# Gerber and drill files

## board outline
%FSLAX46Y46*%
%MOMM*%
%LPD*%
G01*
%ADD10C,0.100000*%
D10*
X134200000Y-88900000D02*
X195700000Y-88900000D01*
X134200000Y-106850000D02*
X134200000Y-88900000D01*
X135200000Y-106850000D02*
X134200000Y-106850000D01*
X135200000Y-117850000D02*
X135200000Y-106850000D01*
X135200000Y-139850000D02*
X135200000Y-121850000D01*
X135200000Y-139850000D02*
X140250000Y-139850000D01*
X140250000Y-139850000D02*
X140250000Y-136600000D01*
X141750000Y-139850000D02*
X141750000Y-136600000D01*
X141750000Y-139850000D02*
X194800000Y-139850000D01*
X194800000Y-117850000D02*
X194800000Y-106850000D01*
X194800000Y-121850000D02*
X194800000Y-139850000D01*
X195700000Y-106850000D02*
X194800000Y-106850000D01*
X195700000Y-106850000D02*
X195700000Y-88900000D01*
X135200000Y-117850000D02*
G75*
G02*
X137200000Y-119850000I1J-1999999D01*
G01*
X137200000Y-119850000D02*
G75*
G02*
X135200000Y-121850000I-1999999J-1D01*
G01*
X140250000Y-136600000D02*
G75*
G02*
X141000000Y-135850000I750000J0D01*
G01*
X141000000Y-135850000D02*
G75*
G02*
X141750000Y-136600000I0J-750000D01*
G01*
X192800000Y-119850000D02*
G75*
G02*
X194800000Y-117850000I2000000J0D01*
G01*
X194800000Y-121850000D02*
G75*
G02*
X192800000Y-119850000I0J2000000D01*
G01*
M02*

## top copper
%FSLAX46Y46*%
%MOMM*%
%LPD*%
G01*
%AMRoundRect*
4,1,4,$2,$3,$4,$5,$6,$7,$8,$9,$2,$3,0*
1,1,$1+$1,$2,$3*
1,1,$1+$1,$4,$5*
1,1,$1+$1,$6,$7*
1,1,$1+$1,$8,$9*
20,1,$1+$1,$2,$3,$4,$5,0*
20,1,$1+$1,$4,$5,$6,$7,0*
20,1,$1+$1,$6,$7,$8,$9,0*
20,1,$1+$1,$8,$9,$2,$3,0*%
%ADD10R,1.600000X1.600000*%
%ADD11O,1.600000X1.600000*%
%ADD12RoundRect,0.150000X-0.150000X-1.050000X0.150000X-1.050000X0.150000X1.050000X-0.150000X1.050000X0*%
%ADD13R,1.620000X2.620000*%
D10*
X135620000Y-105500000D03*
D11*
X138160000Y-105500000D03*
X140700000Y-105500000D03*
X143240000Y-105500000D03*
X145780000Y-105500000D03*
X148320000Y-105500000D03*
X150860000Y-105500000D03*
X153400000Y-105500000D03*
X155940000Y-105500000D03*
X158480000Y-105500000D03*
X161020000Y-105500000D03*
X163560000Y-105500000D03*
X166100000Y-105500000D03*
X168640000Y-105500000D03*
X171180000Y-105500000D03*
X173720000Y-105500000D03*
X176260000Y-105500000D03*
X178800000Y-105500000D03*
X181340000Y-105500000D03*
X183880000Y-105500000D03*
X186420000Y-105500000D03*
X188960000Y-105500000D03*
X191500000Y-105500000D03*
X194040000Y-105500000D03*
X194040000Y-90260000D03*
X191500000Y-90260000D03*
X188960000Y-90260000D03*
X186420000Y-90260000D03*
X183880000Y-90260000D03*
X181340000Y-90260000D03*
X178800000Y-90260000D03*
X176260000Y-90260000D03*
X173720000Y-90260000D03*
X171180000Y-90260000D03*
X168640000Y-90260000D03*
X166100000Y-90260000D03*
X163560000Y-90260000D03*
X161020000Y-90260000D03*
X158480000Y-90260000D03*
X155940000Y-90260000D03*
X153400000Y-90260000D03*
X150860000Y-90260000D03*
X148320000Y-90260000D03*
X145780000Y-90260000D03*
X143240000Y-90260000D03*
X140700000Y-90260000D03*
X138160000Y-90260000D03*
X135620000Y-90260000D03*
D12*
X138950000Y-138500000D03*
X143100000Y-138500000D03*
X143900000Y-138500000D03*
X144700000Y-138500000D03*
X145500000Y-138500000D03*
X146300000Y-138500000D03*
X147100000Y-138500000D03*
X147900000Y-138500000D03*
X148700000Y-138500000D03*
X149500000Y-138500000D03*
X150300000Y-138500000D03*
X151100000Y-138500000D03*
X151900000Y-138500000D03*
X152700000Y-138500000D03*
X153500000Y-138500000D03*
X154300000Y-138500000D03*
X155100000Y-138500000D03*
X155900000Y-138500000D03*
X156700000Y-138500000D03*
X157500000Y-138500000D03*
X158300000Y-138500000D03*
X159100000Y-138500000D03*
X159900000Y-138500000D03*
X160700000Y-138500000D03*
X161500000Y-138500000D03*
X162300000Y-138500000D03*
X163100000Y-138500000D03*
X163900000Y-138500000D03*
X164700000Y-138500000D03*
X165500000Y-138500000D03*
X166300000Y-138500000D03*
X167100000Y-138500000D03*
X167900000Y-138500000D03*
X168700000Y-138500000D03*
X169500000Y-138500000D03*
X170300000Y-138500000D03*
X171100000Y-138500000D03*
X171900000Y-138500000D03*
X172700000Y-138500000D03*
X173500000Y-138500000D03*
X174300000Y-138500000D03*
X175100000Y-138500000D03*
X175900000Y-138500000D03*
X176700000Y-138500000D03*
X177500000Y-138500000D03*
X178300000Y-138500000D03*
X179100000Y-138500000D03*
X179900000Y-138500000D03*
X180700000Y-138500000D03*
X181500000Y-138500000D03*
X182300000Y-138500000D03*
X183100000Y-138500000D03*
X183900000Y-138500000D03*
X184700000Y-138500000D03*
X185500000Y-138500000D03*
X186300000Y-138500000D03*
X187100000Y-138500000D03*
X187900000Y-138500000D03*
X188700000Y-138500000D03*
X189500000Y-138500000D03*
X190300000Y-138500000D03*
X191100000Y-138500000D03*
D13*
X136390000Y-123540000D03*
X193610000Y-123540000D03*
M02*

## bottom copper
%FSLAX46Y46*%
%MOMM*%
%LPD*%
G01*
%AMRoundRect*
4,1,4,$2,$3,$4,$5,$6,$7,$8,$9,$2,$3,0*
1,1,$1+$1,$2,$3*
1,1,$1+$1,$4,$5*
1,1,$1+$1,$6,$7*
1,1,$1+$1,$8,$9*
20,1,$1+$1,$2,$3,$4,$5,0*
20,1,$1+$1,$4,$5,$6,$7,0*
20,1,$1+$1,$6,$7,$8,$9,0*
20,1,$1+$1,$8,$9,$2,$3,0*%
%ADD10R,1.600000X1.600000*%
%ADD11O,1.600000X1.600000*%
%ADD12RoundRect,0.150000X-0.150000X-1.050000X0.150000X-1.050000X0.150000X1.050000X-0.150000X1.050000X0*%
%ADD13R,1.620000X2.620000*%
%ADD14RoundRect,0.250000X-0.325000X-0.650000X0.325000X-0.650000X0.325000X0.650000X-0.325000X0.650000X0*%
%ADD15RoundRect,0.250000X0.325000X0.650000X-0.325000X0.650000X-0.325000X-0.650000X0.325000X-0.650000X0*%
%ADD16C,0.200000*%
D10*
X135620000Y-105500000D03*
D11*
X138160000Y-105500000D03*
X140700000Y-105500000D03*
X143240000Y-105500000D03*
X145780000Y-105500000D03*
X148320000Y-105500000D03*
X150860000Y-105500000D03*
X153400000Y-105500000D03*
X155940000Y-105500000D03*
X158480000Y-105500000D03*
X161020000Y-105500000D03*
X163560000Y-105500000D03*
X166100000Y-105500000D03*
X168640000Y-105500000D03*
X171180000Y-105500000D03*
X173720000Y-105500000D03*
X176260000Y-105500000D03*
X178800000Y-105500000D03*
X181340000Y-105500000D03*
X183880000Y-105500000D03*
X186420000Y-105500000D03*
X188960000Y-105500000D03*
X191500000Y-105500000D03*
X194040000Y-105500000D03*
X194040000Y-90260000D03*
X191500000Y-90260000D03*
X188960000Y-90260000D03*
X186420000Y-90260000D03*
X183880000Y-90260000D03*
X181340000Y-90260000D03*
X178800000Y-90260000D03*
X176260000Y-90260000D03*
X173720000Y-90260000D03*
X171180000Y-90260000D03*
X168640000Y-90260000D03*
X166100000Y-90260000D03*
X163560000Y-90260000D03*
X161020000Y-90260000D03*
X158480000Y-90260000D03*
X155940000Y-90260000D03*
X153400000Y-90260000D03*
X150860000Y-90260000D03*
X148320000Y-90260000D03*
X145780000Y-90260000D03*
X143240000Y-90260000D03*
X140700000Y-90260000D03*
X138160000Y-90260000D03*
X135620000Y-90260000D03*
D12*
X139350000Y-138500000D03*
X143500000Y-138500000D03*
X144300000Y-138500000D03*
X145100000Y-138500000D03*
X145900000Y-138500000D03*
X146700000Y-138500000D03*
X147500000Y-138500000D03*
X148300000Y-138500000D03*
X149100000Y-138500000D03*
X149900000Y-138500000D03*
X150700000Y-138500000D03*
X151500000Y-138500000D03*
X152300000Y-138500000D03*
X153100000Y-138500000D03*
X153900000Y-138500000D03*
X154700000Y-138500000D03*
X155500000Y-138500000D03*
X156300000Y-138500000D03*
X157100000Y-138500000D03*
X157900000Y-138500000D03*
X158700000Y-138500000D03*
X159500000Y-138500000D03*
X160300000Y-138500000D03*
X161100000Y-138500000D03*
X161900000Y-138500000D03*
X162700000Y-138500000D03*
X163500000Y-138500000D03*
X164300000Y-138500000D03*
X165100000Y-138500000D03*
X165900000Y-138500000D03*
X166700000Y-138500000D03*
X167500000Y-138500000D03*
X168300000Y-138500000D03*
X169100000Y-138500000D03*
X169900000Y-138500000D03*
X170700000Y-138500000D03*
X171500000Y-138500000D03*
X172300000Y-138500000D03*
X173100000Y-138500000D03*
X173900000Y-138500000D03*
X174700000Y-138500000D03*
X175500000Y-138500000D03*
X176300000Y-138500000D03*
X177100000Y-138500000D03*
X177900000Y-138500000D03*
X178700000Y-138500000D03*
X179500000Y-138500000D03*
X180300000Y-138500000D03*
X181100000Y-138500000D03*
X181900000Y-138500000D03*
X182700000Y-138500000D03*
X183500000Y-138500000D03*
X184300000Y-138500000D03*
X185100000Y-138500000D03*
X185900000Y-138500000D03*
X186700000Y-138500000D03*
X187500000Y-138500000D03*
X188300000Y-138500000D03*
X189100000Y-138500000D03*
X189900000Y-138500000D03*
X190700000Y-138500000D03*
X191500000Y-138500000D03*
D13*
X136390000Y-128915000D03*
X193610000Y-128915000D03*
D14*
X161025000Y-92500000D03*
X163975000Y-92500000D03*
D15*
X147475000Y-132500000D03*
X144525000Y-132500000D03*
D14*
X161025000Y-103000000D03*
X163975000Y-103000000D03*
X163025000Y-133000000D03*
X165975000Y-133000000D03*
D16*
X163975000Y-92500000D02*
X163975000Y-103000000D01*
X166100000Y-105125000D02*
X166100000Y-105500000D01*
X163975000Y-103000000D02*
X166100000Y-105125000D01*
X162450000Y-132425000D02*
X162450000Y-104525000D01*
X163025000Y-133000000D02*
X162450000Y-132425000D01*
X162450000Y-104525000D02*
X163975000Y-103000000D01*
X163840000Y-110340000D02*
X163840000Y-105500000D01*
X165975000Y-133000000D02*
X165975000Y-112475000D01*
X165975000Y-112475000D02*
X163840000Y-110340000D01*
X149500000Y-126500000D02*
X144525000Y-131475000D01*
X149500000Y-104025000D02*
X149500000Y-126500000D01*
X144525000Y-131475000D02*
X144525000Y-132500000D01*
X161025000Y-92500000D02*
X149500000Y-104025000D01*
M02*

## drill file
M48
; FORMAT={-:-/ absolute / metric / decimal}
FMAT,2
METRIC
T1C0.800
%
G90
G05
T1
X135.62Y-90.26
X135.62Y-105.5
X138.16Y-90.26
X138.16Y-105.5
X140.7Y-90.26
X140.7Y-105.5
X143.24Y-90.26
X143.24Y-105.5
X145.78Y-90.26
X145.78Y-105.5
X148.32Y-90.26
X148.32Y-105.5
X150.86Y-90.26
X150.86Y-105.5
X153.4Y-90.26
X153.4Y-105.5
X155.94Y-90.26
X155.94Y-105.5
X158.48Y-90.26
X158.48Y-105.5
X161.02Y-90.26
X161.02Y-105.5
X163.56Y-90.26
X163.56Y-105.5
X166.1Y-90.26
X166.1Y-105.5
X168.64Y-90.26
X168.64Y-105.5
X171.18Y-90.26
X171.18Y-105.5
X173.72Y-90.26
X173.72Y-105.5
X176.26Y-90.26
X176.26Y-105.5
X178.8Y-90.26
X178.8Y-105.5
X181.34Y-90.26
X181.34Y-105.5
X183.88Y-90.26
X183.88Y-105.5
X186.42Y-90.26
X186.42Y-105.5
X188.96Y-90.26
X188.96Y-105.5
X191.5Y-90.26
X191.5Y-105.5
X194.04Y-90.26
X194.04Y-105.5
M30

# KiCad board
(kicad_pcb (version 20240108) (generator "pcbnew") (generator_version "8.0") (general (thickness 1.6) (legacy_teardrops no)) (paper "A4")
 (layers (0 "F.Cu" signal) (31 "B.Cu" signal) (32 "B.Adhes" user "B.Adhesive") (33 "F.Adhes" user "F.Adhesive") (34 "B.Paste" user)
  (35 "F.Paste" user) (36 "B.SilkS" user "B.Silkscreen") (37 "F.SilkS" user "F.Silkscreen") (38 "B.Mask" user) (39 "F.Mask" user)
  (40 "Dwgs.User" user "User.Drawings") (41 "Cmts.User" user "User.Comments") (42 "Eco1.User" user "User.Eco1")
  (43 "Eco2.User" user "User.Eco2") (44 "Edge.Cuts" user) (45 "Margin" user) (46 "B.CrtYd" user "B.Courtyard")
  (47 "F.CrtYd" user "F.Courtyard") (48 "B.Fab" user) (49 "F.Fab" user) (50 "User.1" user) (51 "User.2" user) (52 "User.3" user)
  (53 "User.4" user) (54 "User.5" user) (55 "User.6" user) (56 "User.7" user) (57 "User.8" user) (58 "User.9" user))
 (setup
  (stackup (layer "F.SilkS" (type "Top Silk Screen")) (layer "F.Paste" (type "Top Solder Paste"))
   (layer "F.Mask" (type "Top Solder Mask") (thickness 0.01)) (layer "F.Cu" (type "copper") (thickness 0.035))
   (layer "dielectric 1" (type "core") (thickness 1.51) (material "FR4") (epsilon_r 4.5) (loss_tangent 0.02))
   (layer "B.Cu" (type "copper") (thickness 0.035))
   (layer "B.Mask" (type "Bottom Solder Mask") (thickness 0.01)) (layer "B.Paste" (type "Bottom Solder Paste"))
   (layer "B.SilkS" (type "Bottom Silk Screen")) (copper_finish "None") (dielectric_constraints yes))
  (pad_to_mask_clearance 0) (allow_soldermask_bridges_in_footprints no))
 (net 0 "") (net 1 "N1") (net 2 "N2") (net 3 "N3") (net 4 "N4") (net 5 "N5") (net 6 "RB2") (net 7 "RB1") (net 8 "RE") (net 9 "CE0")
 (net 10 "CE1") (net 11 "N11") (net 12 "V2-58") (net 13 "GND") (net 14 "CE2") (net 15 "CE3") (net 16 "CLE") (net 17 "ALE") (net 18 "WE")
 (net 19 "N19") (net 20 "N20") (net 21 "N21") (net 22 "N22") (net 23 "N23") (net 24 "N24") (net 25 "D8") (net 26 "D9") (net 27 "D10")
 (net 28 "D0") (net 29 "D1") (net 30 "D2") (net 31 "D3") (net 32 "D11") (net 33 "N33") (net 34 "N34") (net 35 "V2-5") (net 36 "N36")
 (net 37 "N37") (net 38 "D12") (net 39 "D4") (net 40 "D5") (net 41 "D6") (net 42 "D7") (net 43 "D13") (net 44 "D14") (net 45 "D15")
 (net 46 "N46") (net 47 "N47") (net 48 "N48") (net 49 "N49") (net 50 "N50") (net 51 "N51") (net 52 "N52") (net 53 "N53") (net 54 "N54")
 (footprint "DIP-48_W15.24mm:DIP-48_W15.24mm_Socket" (layer "F.Cu") (at 135.62 105.5 90)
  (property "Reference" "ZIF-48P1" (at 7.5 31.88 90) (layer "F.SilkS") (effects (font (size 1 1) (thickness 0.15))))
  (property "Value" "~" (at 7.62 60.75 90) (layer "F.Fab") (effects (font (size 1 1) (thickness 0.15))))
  (pad "1" thru_hole rect (at 0 0 90) (size 1.6 1.6) (drill 0.8) (layers "*.Cu" "*.Mask") (remove_unused_layers no) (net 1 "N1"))
  (pad "2" thru_hole oval (at 0 2.54 90) (size 1.6 1.6) (drill 0.8) (layers "*.Cu" "*.Mask") (remove_unused_layers no) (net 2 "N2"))
  (pad "3" thru_hole oval (at 0 5.08 90) (size 1.6 1.6) (drill 0.8) (layers "*.Cu" "*.Mask") (remove_unused_layers no) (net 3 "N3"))
  (pad "4" thru_hole oval (at 0 7.62 90) (size 1.6 1.6) (drill 0.8) (layers "*.Cu" "*.Mask") (remove_unused_layers no) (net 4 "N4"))
  (pad "5" thru_hole oval (at 0 10.16 90) (size 1.6 1.6) (drill 0.8) (layers "*.Cu" "*.Mask") (remove_unused_layers no) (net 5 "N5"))
  (pad "6" thru_hole oval (at 0 12.7 90) (size 1.6 1.6) (drill 0.8) (layers "*.Cu" "*.Mask") (remove_unused_layers no) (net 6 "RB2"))
  (pad "7" thru_hole oval (at 0 15.24 90) (size 1.6 1.6) (drill 0.8) (layers "*.Cu" "*.Mask") (remove_unused_layers no) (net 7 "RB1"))
  (pad "8" thru_hole oval (at 0 17.78 90) (size 1.6 1.6) (drill 0.8) (layers "*.Cu" "*.Mask") (remove_unused_layers no) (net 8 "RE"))
  (pad "9" thru_hole oval (at 0 20.32 90) (size 1.6 1.6) (drill 0.8) (layers "*.Cu" "*.Mask") (remove_unused_layers no) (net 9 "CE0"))
  (pad "10" thru_hole oval (at 0 22.86 90) (size 1.6 1.6) (drill 0.8) (layers "*.Cu" "*.Mask") (remove_unused_layers no) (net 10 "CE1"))
  (pad "11" thru_hole oval (at 0 25.4 90) (size 1.6 1.6) (drill 0.8) (layers "*.Cu" "*.Mask") (remove_unused_layers no) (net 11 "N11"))
  (pad "12" thru_hole oval (at 0 27.94 90) (size 1.6 1.6) (drill 0.8) (layers "*.Cu" "*.Mask") (remove_unused_layers no) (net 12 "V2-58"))
  (pad "13" thru_hole oval (at 0 30.48 90) (size 1.6 1.6) (drill 0.8) (layers "*.Cu" "*.Mask") (remove_unused_layers no) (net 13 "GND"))
  (pad "14" thru_hole oval (at 0 33.02 90) (size 1.6 1.6) (drill 0.8) (layers "*.Cu" "*.Mask") (remove_unused_layers no) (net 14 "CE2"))
  (pad "15" thru_hole oval (at 0 35.56 90) (size 1.6 1.6) (drill 0.8) (layers "*.Cu" "*.Mask") (remove_unused_layers no) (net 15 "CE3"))
  (pad "16" thru_hole oval (at 0 38.1 90) (size 1.6 1.6) (drill 0.8) (layers "*.Cu" "*.Mask") (remove_unused_layers no) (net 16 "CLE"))
  (pad "17" thru_hole oval (at 0 40.64 90) (size 1.6 1.6) (drill 0.8) (layers "*.Cu" "*.Mask") (remove_unused_layers no) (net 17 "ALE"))
  (pad "18" thru_hole oval (at 0 43.18 90) (size 1.6 1.6) (drill 0.8) (layers "*.Cu" "*.Mask") (remove_unused_layers no) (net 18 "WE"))
  (pad "19" thru_hole oval (at 0 45.72 90) (size 1.6 1.6) (drill 0.8) (layers "*.Cu" "*.Mask") (remove_unused_layers no) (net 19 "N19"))
  (pad "20" thru_hole oval (at 0 48.26 90) (size 1.6 1.6) (drill 0.8) (layers "*.Cu" "*.Mask") (remove_unused_layers no) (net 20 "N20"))
  (pad "21" thru_hole oval (at 0 50.8 90) (size 1.6 1.6) (drill 0.8) (layers "*.Cu" "*.Mask") (remove_unused_layers no) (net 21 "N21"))
  (pad "22" thru_hole oval (at 0 53.34 90) (size 1.6 1.6) (drill 0.8) (layers "*.Cu" "*.Mask") (remove_unused_layers no) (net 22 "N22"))
  (pad "23" thru_hole oval (at 0 55.88 90) (size 1.6 1.6) (drill 0.8) (layers "*.Cu" "*.Mask") (remove_unused_layers no) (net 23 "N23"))
  (pad "24" thru_hole oval (at 0 58.42 90) (size 1.6 1.6) (drill 0.8) (layers "*.Cu" "*.Mask") (remove_unused_layers no) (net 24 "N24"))
  (pad "25" thru_hole oval (at 15.24 58.42 90) (size 1.6 1.6) (drill 0.8) (layers "*.Cu" "*.Mask") (remove_unused_layers no) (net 13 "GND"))
  (pad "26" thru_hole oval (at 15.24 55.88 90) (size 1.6 1.6) (drill 0.8) (layers "*.Cu" "*.Mask") (remove_unused_layers no) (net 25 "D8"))
  (pad "27" thru_hole oval (at 15.24 53.34 90) (size 1.6 1.6) (drill 0.8) (layers "*.Cu" "*.Mask") (remove_unused_layers no) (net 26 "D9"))
  (pad "28" thru_hole oval (at 15.24 50.8 90) (size 1.6 1.6) (drill 0.8) (layers "*.Cu" "*.Mask") (remove_unused_layers no) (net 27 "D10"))
  (pad "29" thru_hole oval (at 15.24 48.26 90) (size 1.6 1.6) (drill 0.8) (layers "*.Cu" "*.Mask") (remove_unused_layers no) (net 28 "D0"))
  (pad "30" thru_hole oval (at 15.24 45.72 90) (size 1.6 1.6) (drill 0.8) (layers "*.Cu" "*.Mask") (remove_unused_layers no) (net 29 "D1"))
  (pad "31" thru_hole oval (at 15.24 43.18 90) (size 1.6 1.6) (drill 0.8) (layers "*.Cu" "*.Mask") (remove_unused_layers no) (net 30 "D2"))
  (pad "32" thru_hole oval (at 15.24 40.64 90) (size 1.6 1.6) (drill 0.8) (layers "*.Cu" "*.Mask") (remove_unused_layers no) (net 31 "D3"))
  (pad "33" thru_hole oval (at 15.24 38.1 90) (size 1.6 1.6) (drill 0.8) (layers "*.Cu" "*.Mask") (remove_unused_layers no) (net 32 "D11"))
  (pad "34" thru_hole oval (at 15.24 35.56 90) (size 1.6 1.6) (drill 0.8) (layers "*.Cu" "*.Mask") (remove_unused_layers no) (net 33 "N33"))
  (pad "35" thru_hole oval (at 15.24 33.02 90) (size 1.6 1.6) (drill 0.8) (layers "*.Cu" "*.Mask") (remove_unused_layers no) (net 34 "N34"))
  (pad "36" thru_hole oval (at 15.24 30.48 90) (size 1.6 1.6) (drill 0.8) (layers "*.Cu" "*.Mask") (remove_unused_layers no) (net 13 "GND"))
  (pad "37" thru_hole oval (at 15.24 27.94 90) (size 1.6 1.6) (drill 0.8) (layers "*.Cu" "*.Mask") (remove_unused_layers no) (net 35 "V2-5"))
  (pad "38" thru_hole oval (at 15.24 25.4 90) (size 1.6 1.6) (drill 0.8) (layers "*.Cu" "*.Mask") (remove_unused_layers no) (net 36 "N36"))
  (pad "39" thru_hole oval (at 15.24 22.86 90) (size 1.6 1.6) (drill 0.8) (layers "*.Cu" "*.Mask") (remove_unused_layers no) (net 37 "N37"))
  (pad "40" thru_hole oval (at 15.24 20.32 90) (size 1.6 1.6) (drill 0.8) (layers "*.Cu" "*.Mask") (remove_unused_layers no) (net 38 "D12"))
  (pad "41" thru_hole oval (at 15.24 17.78 90) (size 1.6 1.6) (drill 0.8) (layers "*.Cu" "*.Mask") (remove_unused_layers no) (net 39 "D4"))
  (pad "42" thru_hole oval (at 15.24 15.24 90) (size 1.6 1.6) (drill 0.8) (layers "*.Cu" "*.Mask") (remove_unused_layers no) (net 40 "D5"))
  (pad "43" thru_hole oval (at 15.24 12.7 90) (size 1.6 1.6) (drill 0.8) (layers "*.Cu" "*.Mask") (remove_unused_layers no) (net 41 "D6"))
  (pad "44" thru_hole oval (at 15.24 10.16 90) (size 1.6 1.6) (drill 0.8) (layers "*.Cu" "*.Mask") (remove_unused_layers no) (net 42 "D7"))
  (pad "45" thru_hole oval (at 15.24 7.62 90) (size 1.6 1.6) (drill 0.8) (layers "*.Cu" "*.Mask") (remove_unused_layers no) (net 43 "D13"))
  (pad "46" thru_hole oval (at 15.24 5.08 90) (size 1.6 1.6) (drill 0.8) (layers "*.Cu" "*.Mask") (remove_unused_layers no) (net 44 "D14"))
  (pad "47" thru_hole oval (at 15.24 2.54 90) (size 1.6 1.6) (drill 0.8) (layers "*.Cu" "*.Mask") (remove_unused_layers no) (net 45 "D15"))
  (pad "48" thru_hole oval (at 15.24 0 90) (size 1.6 1.6) (drill 0.8) (layers "*.Cu" "*.Mask") (remove_unused_layers no) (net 13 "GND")))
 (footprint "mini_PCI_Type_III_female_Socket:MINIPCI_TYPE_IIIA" (layer "F.Cu") (at 135.2 139.85)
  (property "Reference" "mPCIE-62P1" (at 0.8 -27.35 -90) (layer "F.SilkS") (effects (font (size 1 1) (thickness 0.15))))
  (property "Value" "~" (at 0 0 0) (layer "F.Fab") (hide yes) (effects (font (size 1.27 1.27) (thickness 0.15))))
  (fp_line (start -1 -50.95) (end 60.5 -50.95) (stroke (width 0.1) (type solid)) (layer "Edge.Cuts"))
  (fp_line (start -1 -33) (end -1 -50.95) (stroke (width 0.1) (type solid)) (layer "Edge.Cuts"))
  (fp_line (start 0 -33) (end -1 -33) (stroke (width 0.1) (type solid)) (layer "Edge.Cuts"))
  (fp_line (start 0 -22) (end 0 -33) (stroke (width 0.1) (type solid)) (layer "Edge.Cuts"))
  (fp_line (start 0 0) (end 0 -18) (stroke (width 0.1) (type solid)) (layer "Edge.Cuts"))
  (fp_line (start 0 0) (end 5.05 0) (stroke (width 0.1) (type solid)) (layer "Edge.Cuts"))
  (fp_line (start 5.05 0) (end 5.05 -3.25) (stroke (width 0.1) (type solid)) (layer "Edge.Cuts"))
  (fp_line (start 6.55 0) (end 6.55 -3.25) (stroke (width 0.1) (type solid)) (layer "Edge.Cuts"))
  (fp_line (start 6.55 0) (end 59.6 0) (stroke (width 0.1) (type solid)) (layer "Edge.Cuts"))
  (fp_line (start 59.6 -22) (end 59.6 -33) (stroke (width 0.1) (type solid)) (layer "Edge.Cuts"))
  (fp_line (start 59.6 -18) (end 59.6 0) (stroke (width 0.1) (type solid)) (layer "Edge.Cuts"))
  (fp_line (start 60.5 -33) (end 59.6 -33) (stroke (width 0.1) (type solid)) (layer "Edge.Cuts"))
  (fp_line (start 60.5 -33) (end 60.5 -50.95) (stroke (width 0.1) (type solid)) (layer "Edge.Cuts"))
  (fp_arc (start 0 -22) (mid 1.414214 -21.414214) (end 2 -20) (stroke (width 0.1) (type solid)) (layer "Edge.Cuts"))
  (fp_arc (start 2 -20) (mid 1.414214 -18.585786) (end 0 -18) (stroke (width 0.1) (type solid)) (layer "Edge.Cuts"))
  (fp_arc (start 5.05 -3.25) (mid 5.26967 -3.78033) (end 5.8 -4) (stroke (width 0.1) (type solid)) (layer "Edge.Cuts"))
  (fp_arc (start 5.8 -4) (mid 6.33033 -3.78033) (end 6.55 -3.25) (stroke (width 0.1) (type solid)) (layer "Edge.Cuts"))
  (fp_arc (start 57.6 -20) (mid 58.185786 -21.414214) (end 59.6 -22) (stroke (width 0.1) (type solid)) (layer "Edge.Cuts"))
  (fp_arc (start 59.6 -18) (mid 58.185786 -18.585786) (end 57.6 -20) (stroke (width 0.1) (type solid)) (layer "Edge.Cuts"))
  (pad "1" smd roundrect (at 3.75 -1.35) (size 0.6 2.4) (layers "F.Cu") (roundrect_rratio 0.25) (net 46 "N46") (solder_mask_margin 0.1016)
   (thermal_bridge_angle 0))
  (pad "1" smd roundrect (at 4.15 -1.35) (size 0.6 2.4) (layers "B.Cu") (roundrect_rratio 0.25) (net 46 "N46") (solder_mask_margin 0.1016)
   (thermal_bridge_angle 0))
  (pad "2" smd roundrect (at 7.9 -1.35) (size 0.6 2.4) (layers "F.Cu") (roundrect_rratio 0.25) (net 2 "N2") (solder_mask_margin 0.1016)
   (thermal_bridge_angle 0))
  (pad "2" smd roundrect (at 8.3 -1.35) (size 0.6 2.4) (layers "B.Cu") (roundrect_rratio 0.25) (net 2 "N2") (solder_mask_margin 0.1016)
   (thermal_bridge_angle 0))
  (pad "3" smd roundrect (at 8.7 -1.35) (size 0.6 2.4) (layers "F.Cu") (roundrect_rratio 0.25) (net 3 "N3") (solder_mask_margin 0.1016)
   (thermal_bridge_angle 0))
  (pad "3" smd roundrect (at 9.1 -1.35) (size 0.6 2.4) (layers "B.Cu") (roundrect_rratio 0.25) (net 3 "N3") (solder_mask_margin 0.1016)
   (thermal_bridge_angle 0))
  (pad "4" smd roundrect (at 9.5 -1.35) (size 0.6 2.4) (layers "F.Cu") (roundrect_rratio 0.25) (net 4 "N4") (solder_mask_margin 0.1016)
   (thermal_bridge_angle 0))
  (pad "4" smd roundrect (at 9.9 -1.35) (size 0.6 2.4) (layers "B.Cu") (roundrect_rratio 0.25) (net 4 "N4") (solder_mask_margin 0.1016)
   (thermal_bridge_angle 0))
  (pad "5" smd roundrect (at 10.3 -1.35) (size 0.6 2.4) (layers "F.Cu") (roundrect_rratio 0.25) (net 35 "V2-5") (solder_mask_margin 0.1016)
   (thermal_bridge_angle 0))
  (pad "5" smd roundrect (at 10.7 -1.35) (size 0.6 2.4) (layers "B.Cu") (roundrect_rratio 0.25) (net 35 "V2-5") (solder_mask_margin 0.1016)
   (thermal_bridge_angle 0))
  (pad "6" smd roundrect (at 11.1 -1.35) (size 0.6 2.4) (layers "F.Cu") (roundrect_rratio 0.25) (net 13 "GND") (solder_mask_margin 0.1016)
   (thermal_bridge_angle 0))
  (pad "6" smd roundrect (at 11.5 -1.35) (size 0.6 2.4) (layers "B.Cu") (roundrect_rratio 0.25) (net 13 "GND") (solder_mask_margin 0.1016)
   (thermal_bridge_angle 0))
  (pad "7" smd roundrect (at 11.9 -1.35) (size 0.6 2.4) (layers "F.Cu") (roundrect_rratio 0.25) (solder_mask_margin 0.1016)
   (thermal_bridge_angle 0))
  (pad "7" smd roundrect (at 12.3 -1.35) (size 0.6 2.4) (layers "B.Cu") (roundrect_rratio 0.25) (solder_mask_margin 0.1016)
   (thermal_bridge_angle 0))
  (pad "8" smd roundrect (at 12.7 -1.35) (size 0.6 2.4) (layers "F.Cu") (roundrect_rratio 0.25) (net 13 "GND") (solder_mask_margin 0.1016)
   (thermal_bridge_angle 0))
  (pad "8" smd roundrect (at 13.1 -1.35) (size 0.6 2.4) (layers "B.Cu") (roundrect_rratio 0.25) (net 13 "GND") (solder_mask_margin 0.1016)
   (thermal_bridge_angle 0))
  (pad "9" smd roundrect (at 13.5 -1.35) (size 0.6 2.4) (layers "F.Cu") (roundrect_rratio 0.25) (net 13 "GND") (solder_mask_margin 0.1016)
   (thermal_bridge_angle 0))
  (pad "9" smd roundrect (at 13.9 -1.35) (size 0.6 2.4) (layers "B.Cu") (roundrect_rratio 0.25) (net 13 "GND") (solder_mask_margin 0.1016)
   (thermal_bridge_angle 0))
  (pad "10" smd roundrect (at 14.3 -1.35) (size 0.6 2.4) (layers "F.Cu") (roundrect_rratio 0.25) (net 13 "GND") (solder_mask_margin 0.1016)
   (thermal_bridge_angle 0))
  (pad "10" smd roundrect (at 14.7 -1.35) (size 0.6 2.4) (layers "B.Cu") (roundrect_rratio 0.25) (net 13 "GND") (solder_mask_margin 0.1016)
   (thermal_bridge_angle 0))
  (pad "11" smd roundrect (at 15.1 -1.35) (size 0.6 2.4) (layers "F.Cu") (roundrect_rratio 0.25) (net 11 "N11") (solder_mask_margin 0.1016)
   (thermal_bridge_angle 0))
  (pad "11" smd roundrect (at 15.5 -1.35) (size 0.6 2.4) (layers "B.Cu") (roundrect_rratio 0.25) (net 11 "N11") (solder_mask_margin 0.1016)
   (thermal_bridge_angle 0))
  (pad "12" smd roundrect (at 15.9 -1.35) (size 0.6 2.4) (layers "F.Cu") (roundrect_rratio 0.25) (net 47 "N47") (solder_mask_margin 0.1016)
   (thermal_bridge_angle 0))
  (pad "12" smd roundrect (at 16.3 -1.35) (size 0.6 2.4) (layers "B.Cu") (roundrect_rratio 0.25) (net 47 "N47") (solder_mask_margin 0.1016)
   (thermal_bridge_angle 0))
  (pad "13" smd roundrect (at 16.7 -1.35) (size 0.6 2.4) (layers "F.Cu") (roundrect_rratio 0.25) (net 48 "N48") (solder_mask_margin 0.1016)
   (thermal_bridge_angle 0))
  (pad "13" smd roundrect (at 17.1 -1.35) (size 0.6 2.4) (layers "B.Cu") (roundrect_rratio 0.25) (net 48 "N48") (solder_mask_margin 0.1016)
   (thermal_bridge_angle 0))
  (pad "14" smd roundrect (at 17.5 -1.35) (size 0.6 2.4) (layers "F.Cu") (roundrect_rratio 0.25) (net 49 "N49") (solder_mask_margin 0.1016)
   (thermal_bridge_angle 0))
  (pad "14" smd roundrect (at 17.9 -1.35) (size 0.6 2.4) (layers "B.Cu") (roundrect_rratio 0.25) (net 49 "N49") (solder_mask_margin 0.1016)
   (thermal_bridge_angle 0))
  (pad "15" smd roundrect (at 18.3 -1.35) (size 0.6 2.4) (layers "F.Cu") (roundrect_rratio 0.25) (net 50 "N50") (solder_mask_margin 0.1016)
   (thermal_bridge_angle 0))
  (pad "15" smd roundrect (at 18.7 -1.35) (size 0.6 2.4) (layers "B.Cu") (roundrect_rratio 0.25) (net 50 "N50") (solder_mask_margin 0.1016)
   (thermal_bridge_angle 0))
  (pad "16" smd roundrect (at 19.1 -1.35) (size 0.6 2.4) (layers "F.Cu") (roundrect_rratio 0.25) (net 13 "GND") (solder_mask_margin 0.1016)
   (thermal_bridge_angle 0))
  (pad "16" smd roundrect (at 19.5 -1.35) (size 0.6 2.4) (layers "B.Cu") (roundrect_rratio 0.25) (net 13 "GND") (solder_mask_margin 0.1016)
   (thermal_bridge_angle 0))
  (pad "17" smd roundrect (at 19.9 -1.35) (size 0.6 2.4) (layers "F.Cu") (roundrect_rratio 0.25) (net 27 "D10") (solder_mask_margin 0.1016)
   (thermal_bridge_angle 0))
  (pad "17" smd roundrect (at 20.3 -1.35) (size 0.6 2.4) (layers "B.Cu") (roundrect_rratio 0.25) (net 27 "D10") (solder_mask_margin 0.1016)
   (thermal_bridge_angle 0))
  (pad "18" smd roundrect (at 20.7 -1.35) (size 0.6 2.4) (layers "F.Cu") (roundrect_rratio 0.25) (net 30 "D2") (solder_mask_margin 0.1016)
   (thermal_bridge_angle 0))
  (pad "18" smd roundrect (at 21.1 -1.35) (size 0.6 2.4) (layers "B.Cu") (roundrect_rratio 0.25) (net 30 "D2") (solder_mask_margin 0.1016)
   (thermal_bridge_angle 0))
  (pad "19" smd roundrect (at 21.5 -1.35) (size 0.6 2.4) (layers "F.Cu") (roundrect_rratio 0.25) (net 13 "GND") (solder_mask_margin 0.1016)
   (thermal_bridge_angle 0))
  (pad "19" smd roundrect (at 21.9 -1.35) (size 0.6 2.4) (layers "B.Cu") (roundrect_rratio 0.25) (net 13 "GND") (solder_mask_margin 0.1016)
   (thermal_bridge_angle 0))
  (pad "20" smd roundrect (at 22.3 -1.35) (size 0.6 2.4) (layers "F.Cu") (roundrect_rratio 0.25) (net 32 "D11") (solder_mask_margin 0.1016)
   (thermal_bridge_angle 0))
  (pad "20" smd roundrect (at 22.7 -1.35) (size 0.6 2.4) (layers "B.Cu") (roundrect_rratio 0.25) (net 32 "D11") (solder_mask_margin 0.1016)
   (thermal_bridge_angle 0))
  (pad "21" smd roundrect (at 23.1 -1.35) (size 0.6 2.4) (layers "F.Cu") (roundrect_rratio 0.25) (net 29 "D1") (solder_mask_margin 0.1016)
   (thermal_bridge_angle 0))
  (pad "21" smd roundrect (at 23.5 -1.35) (size 0.6 2.4) (layers "B.Cu") (roundrect_rratio 0.25) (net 29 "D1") (solder_mask_margin 0.1016)
   (thermal_bridge_angle 0))
  (pad "22" smd roundrect (at 23.9 -1.35) (size 0.6 2.4) (layers "F.Cu") (roundrect_rratio 0.25) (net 13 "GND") (solder_mask_margin 0.1016)
   (thermal_bridge_angle 0))
  (pad "22" smd roundrect (at 24.3 -1.35) (size 0.6 2.4) (layers "B.Cu") (roundrect_rratio 0.25) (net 13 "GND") (solder_mask_margin 0.1016)
   (thermal_bridge_angle 0))
  (pad "23" smd roundrect (at 24.7 -1.35) (size 0.6 2.4) (layers "F.Cu") (roundrect_rratio 0.25) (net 25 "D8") (solder_mask_margin 0.1016)
   (thermal_bridge_angle 0))
  (pad "23" smd roundrect (at 25.1 -1.35) (size 0.6 2.4) (layers "B.Cu") (roundrect_rratio 0.25) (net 25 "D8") (solder_mask_margin 0.1016)
   (thermal_bridge_angle 0))
  (pad "24" smd roundrect (at 25.5 -1.35) (size 0.6 2.4) (layers "F.Cu") (roundrect_rratio 0.25) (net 26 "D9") (solder_mask_margin 0.1016)
   (thermal_bridge_angle 0))
  (pad "24" smd roundrect (at 25.9 -1.35) (size 0.6 2.4) (layers "B.Cu") (roundrect_rratio 0.25) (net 26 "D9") (solder_mask_margin 0.1016)
   (thermal_bridge_angle 0))
  (pad "25" smd roundrect (at 26.3 -1.35) (size 0.6 2.4) (layers "F.Cu") (roundrect_rratio 0.25) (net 13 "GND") (solder_mask_margin 0.1016)
   (thermal_bridge_angle 0))
  (pad "25" smd roundrect (at 26.7 -1.35) (size 0.6 2.4) (layers "B.Cu") (roundrect_rratio 0.25) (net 13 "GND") (solder_mask_margin 0.1016)
   (thermal_bridge_angle 0))
  (pad "26" smd roundrect (at 27.1 -1.35) (size 0.6 2.4) (layers "F.Cu") (roundrect_rratio 0.25) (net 31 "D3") (solder_mask_margin 0.1016)
   (thermal_bridge_angle 0))
  (pad "26" smd roundrect (at 27.5 -1.35) (size 0.6 2.4) (layers "B.Cu") (roundrect_rratio 0.25) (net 31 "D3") (solder_mask_margin 0.1016)
   (thermal_bridge_angle 0))
  (pad "27" smd roundrect (at 27.9 -1.35) (size 0.6 2.4) (layers "F.Cu") (roundrect_rratio 0.25) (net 28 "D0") (solder_mask_margin 0.1016)
   (thermal_bridge_angle 0))
  (pad "27" smd roundrect (at 28.3 -1.35) (size 0.6 2.4) (layers "B.Cu") (roundrect_rratio 0.25) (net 28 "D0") (solder_mask_margin 0.1016)
   (thermal_bridge_angle 0))
  (pad "28" smd roundrect (at 28.7 -1.35) (size 0.6 2.4) (layers "F.Cu") (roundrect_rratio 0.25) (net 13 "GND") (solder_mask_margin 0.1016)
   (thermal_bridge_angle 0))
  (pad "28" smd roundrect (at 29.1 -1.35) (size 0.6 2.4) (layers "B.Cu") (roundrect_rratio 0.25) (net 13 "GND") (solder_mask_margin 0.1016)
   (thermal_bridge_angle 0))
  (pad "29" smd roundrect (at 29.5 -1.35) (size 0.6 2.4) (layers "F.Cu") (roundrect_rratio 0.25) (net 18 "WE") (solder_mask_margin 0.1016)
   (thermal_bridge_angle 0))
  (pad "29" smd roundrect (at 29.9 -1.35) (size 0.6 2.4) (layers "B.Cu") (roundrect_rratio 0.25) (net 18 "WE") (solder_mask_margin 0.1016)
   (thermal_bridge_angle 0))
  (pad "30" smd roundrect (at 30.3 -1.35) (size 0.6 2.4) (layers "F.Cu") (roundrect_rratio 0.25) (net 13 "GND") (solder_mask_margin 0.1016)
   (thermal_bridge_angle 0))
  (pad "30" smd roundrect (at 30.7 -1.35) (size 0.6 2.4) (layers "B.Cu") (roundrect_rratio 0.25) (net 13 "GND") (solder_mask_margin 0.1016)
   (thermal_bridge_angle 0))
  (pad "31" smd roundrect (at 31.1 -1.35) (size 0.6 2.4) (layers "F.Cu") (roundrect_rratio 0.25) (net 16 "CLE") (solder_mask_margin 0.1016)
   (thermal_bridge_angle 0))
  (pad "31" smd roundrect (at 31.5 -1.35) (size 0.6 2.4) (layers "B.Cu") (roundrect_rratio 0.25) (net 16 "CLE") (solder_mask_margin 0.1016)
   (thermal_bridge_angle 0))
  (pad "32" smd roundrect (at 31.9 -1.35) (size 0.6 2.4) (layers "F.Cu") (roundrect_rratio 0.25) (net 13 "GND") (solder_mask_margin 0.1016)
   (thermal_bridge_angle 0))
  (pad "32" smd roundrect (at 32.3 -1.35) (size 0.6 2.4) (layers "B.Cu") (roundrect_rratio 0.25) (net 13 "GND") (solder_mask_margin 0.1016)
   (thermal_bridge_angle 0))
  (pad "33" smd roundrect (at 32.7 -1.35) (size 0.6 2.4) (layers "F.Cu") (roundrect_rratio 0.25) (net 17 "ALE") (solder_mask_margin 0.1016)
   (thermal_bridge_angle 0))
  (pad "33" smd roundrect (at 33.1 -1.35) (size 0.6 2.4) (layers "B.Cu") (roundrect_rratio 0.25) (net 17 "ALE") (solder_mask_margin 0.1016)
   (thermal_bridge_angle 0))
  (pad "34" smd roundrect (at 33.5 -1.35) (size 0.6 2.4) (layers "F.Cu") (roundrect_rratio 0.25) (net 13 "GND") (solder_mask_margin 0.1016)
   (thermal_bridge_angle 0))
  (pad "34" smd roundrect (at 33.9 -1.35) (size 0.6 2.4) (layers "B.Cu") (roundrect_rratio 0.25) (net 13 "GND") (solder_mask_margin 0.1016)
   (thermal_bridge_angle 0))
  (pad "35" smd roundrect (at 34.3 -1.35) (size 0.6 2.4) (layers "F.Cu") (roundrect_rratio 0.25) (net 9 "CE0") (solder_mask_margin 0.1016)
   (thermal_bridge_angle 0))
  (pad "35" smd roundrect (at 34.7 -1.35) (size 0.6 2.4) (layers "B.Cu") (roundrect_rratio 0.25) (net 9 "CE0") (solder_mask_margin 0.1016)
   (thermal_bridge_angle 0))
  (pad "36" smd roundrect (at 35.1 -1.35) (size 0.6 2.4) (layers "F.Cu") (roundrect_rratio 0.25) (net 14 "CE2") (solder_mask_margin 0.1016)
   (thermal_bridge_angle 0))
  (pad "36" smd roundrect (at 35.5 -1.35) (size 0.6 2.4) (layers "B.Cu") (roundrect_rratio 0.25) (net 14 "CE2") (solder_mask_margin 0.1016)
   (thermal_bridge_angle 0))
  (pad "37" smd roundrect (at 35.9 -1.35) (size 0.6 2.4) (layers "F.Cu") (roundrect_rratio 0.25) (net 10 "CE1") (solder_mask_margin 0.1016)
   (thermal_bridge_angle 0))
  (pad "37" smd roundrect (at 36.3 -1.35) (size 0.6 2.4) (layers "B.Cu") (roundrect_rratio 0.25) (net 10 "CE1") (solder_mask_margin 0.1016)
   (thermal_bridge_angle 0))
  (pad "38" smd roundrect (at 36.7 -1.35) (size 0.6 2.4) (layers "F.Cu") (roundrect_rratio 0.25) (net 13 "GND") (solder_mask_margin 0.1016)
   (thermal_bridge_angle 0))
  (pad "38" smd roundrect (at 37.1 -1.35) (size 0.6 2.4) (layers "B.Cu") (roundrect_rratio 0.25) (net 13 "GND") (solder_mask_margin 0.1016)
   (thermal_bridge_angle 0))
  (pad "39" smd roundrect (at 37.5 -1.35) (size 0.6 2.4) (layers "F.Cu") (roundrect_rratio 0.25) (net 8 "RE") (solder_mask_margin 0.1016)
   (thermal_bridge_angle 0))
  (pad "39" smd roundrect (at 37.9 -1.35) (size 0.6 2.4) (layers "B.Cu") (roundrect_rratio 0.25) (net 8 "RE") (solder_mask_margin 0.1016)
   (thermal_bridge_angle 0))
  (pad "40" smd roundrect (at 38.3 -1.35) (size 0.6 2.4) (layers "F.Cu") (roundrect_rratio 0.25) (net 13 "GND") (solder_mask_margin 0.1016)
   (thermal_bridge_angle 0))
  (pad "40" smd roundrect (at 38.7 -1.35) (size 0.6 2.4) (layers "B.Cu") (roundrect_rratio 0.25) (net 13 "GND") (solder_mask_margin 0.1016)
   (thermal_bridge_angle 0))
  (pad "41" smd roundrect (at 39.1 -1.35) (size 0.6 2.4) (layers "F.Cu") (roundrect_rratio 0.25) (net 15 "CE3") (solder_mask_margin 0.1016)
   (thermal_bridge_angle 0))
  (pad "41" smd roundrect (at 39.5 -1.35) (size 0.6 2.4) (layers "B.Cu") (roundrect_rratio 0.25) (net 15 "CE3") (solder_mask_margin 0.1016)
   (thermal_bridge_angle 0))
  (pad "42" smd roundrect (at 39.9 -1.35) (size 0.6 2.4) (layers "F.Cu") (roundrect_rratio 0.25) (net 13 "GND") (solder_mask_margin 0.1016)
   (thermal_bridge_angle 0))
  (pad "42" smd roundrect (at 40.3 -1.35) (size 0.6 2.4) (layers "B.Cu") (roundrect_rratio 0.25) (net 13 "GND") (solder_mask_margin 0.1016)
   (thermal_bridge_angle 0))
  (pad "43" smd roundrect (at 40.7 -1.35) (size 0.6 2.4) (layers "F.Cu") (roundrect_rratio 0.25) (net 7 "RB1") (solder_mask_margin 0.1016)
   (thermal_bridge_angle 0))
  (pad "43" smd roundrect (at 41.1 -1.35) (size 0.6 2.4) (layers "B.Cu") (roundrect_rratio 0.25) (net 7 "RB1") (solder_mask_margin 0.1016)
   (thermal_bridge_angle 0))
  (pad "44" smd roundrect (at 41.5 -1.35) (size 0.6 2.4) (layers "F.Cu") (roundrect_rratio 0.25) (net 6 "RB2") (solder_mask_margin 0.1016)
   (thermal_bridge_angle 0))
  (pad "44" smd roundrect (at 41.9 -1.35) (size 0.6 2.4) (layers "B.Cu") (roundrect_rratio 0.25) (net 6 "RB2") (solder_mask_margin 0.1016)
   (thermal_bridge_angle 0))
  (pad "45" smd roundrect (at 42.3 -1.35) (size 0.6 2.4) (layers "F.Cu") (roundrect_rratio 0.25) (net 13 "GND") (solder_mask_margin 0.1016)
   (thermal_bridge_angle 0))
  (pad "45" smd roundrect (at 42.7 -1.35) (size 0.6 2.4) (layers "B.Cu") (roundrect_rratio 0.25) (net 13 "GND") (solder_mask_margin 0.1016)
   (thermal_bridge_angle 0))
  (pad "46" smd roundrect (at 43.1 -1.35) (size 0.6 2.4) (layers "F.Cu") (roundrect_rratio 0.25) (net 39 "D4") (solder_mask_margin 0.1016)
   (thermal_bridge_angle 0))
  (pad "46" smd roundrect (at 43.5 -1.35) (size 0.6 2.4) (layers "B.Cu") (roundrect_rratio 0.25) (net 39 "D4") (solder_mask_margin 0.1016)
   (thermal_bridge_angle 0))
  (pad "47" smd roundrect (at 43.9 -1.35) (size 0.6 2.4) (layers "F.Cu") (roundrect_rratio 0.25) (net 41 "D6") (solder_mask_margin 0.1016)
   (thermal_bridge_angle 0))
  (pad "47" smd roundrect (at 44.3 -1.35) (size 0.6 2.4) (layers "B.Cu") (roundrect_rratio 0.25) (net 41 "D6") (solder_mask_margin 0.1016)
   (thermal_bridge_angle 0))
  (pad "48" smd roundrect (at 44.7 -1.35) (size 0.6 2.4) (layers "F.Cu") (roundrect_rratio 0.25) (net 13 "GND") (solder_mask_margin 0.1016)
   (thermal_bridge_angle 0))
  (pad "48" smd roundrect (at 45.1 -1.35) (size 0.6 2.4) (layers "B.Cu") (roundrect_rratio 0.25) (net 13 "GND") (solder_mask_margin 0.1016)
   (thermal_bridge_angle 0))
  (pad "49" smd roundrect (at 45.5 -1.35) (size 0.6 2.4) (layers "F.Cu") (roundrect_rratio 0.25) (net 40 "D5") (solder_mask_margin 0.1016)
   (thermal_bridge_angle 0))
  (pad "49" smd roundrect (at 45.9 -1.35) (size 0.6 2.4) (layers "B.Cu") (roundrect_rratio 0.25) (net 40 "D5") (solder_mask_margin 0.1016)
   (thermal_bridge_angle 0))
  (pad "50" smd roundrect (at 46.3 -1.35) (size 0.6 2.4) (layers "F.Cu") (roundrect_rratio 0.25) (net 38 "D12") (solder_mask_margin 0.1016)
   (thermal_bridge_angle 0))
  (pad "50" smd roundrect (at 46.7 -1.35) (size 0.6 2.4) (layers "B.Cu") (roundrect_rratio 0.25) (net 38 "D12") (solder_mask_margin 0.1016)
   (thermal_bridge_angle 0))
  (pad "51" smd roundrect (at 47.1 -1.35) (size 0.6 2.4) (layers "F.Cu") (roundrect_rratio 0.25) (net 13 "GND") (solder_mask_margin 0.1016)
   (thermal_bridge_angle 0))
  (pad "51" smd roundrect (at 47.5 -1.35) (size 0.6 2.4) (layers "B.Cu") (roundrect_rratio 0.25) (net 13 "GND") (solder_mask_margin 0.1016)
   (thermal_bridge_angle 0))
  (pad "52" smd roundrect (at 47.9 -1.35) (size 0.6 2.4) (layers "F.Cu") (roundrect_rratio 0.25) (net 42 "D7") (solder_mask_margin 0.1016)
   (thermal_bridge_angle 0))
  (pad "52" smd roundrect (at 48.3 -1.35) (size 0.6 2.4) (layers "B.Cu") (roundrect_rratio 0.25) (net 42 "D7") (solder_mask_margin 0.1016)
   (thermal_bridge_angle 0))
  (pad "53" smd roundrect (at 48.7 -1.35) (size 0.6 2.4) (layers "F.Cu") (roundrect_rratio 0.25) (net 43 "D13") (solder_mask_margin 0.1016)
   (thermal_bridge_angle 0))
  (pad "53" smd roundrect (at 49.1 -1.35) (size 0.6 2.4) (layers "B.Cu") (roundrect_rratio 0.25) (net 43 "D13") (solder_mask_margin 0.1016)
   (thermal_bridge_angle 0))
  (pad "54" smd roundrect (at 49.5 -1.35) (size 0.6 2.4) (layers "F.Cu") (roundrect_rratio 0.25) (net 13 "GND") (solder_mask_margin 0.1016)
   (thermal_bridge_angle 0))
  (pad "54" smd roundrect (at 49.9 -1.35) (size 0.6 2.4) (layers "B.Cu") (roundrect_rratio 0.25) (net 13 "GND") (solder_mask_margin 0.1016)
   (thermal_bridge_angle 0))
  (pad "55" smd roundrect (at 50.3 -1.35) (size 0.6 2.4) (layers "F.Cu") (roundrect_rratio 0.25) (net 45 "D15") (solder_mask_margin 0.1016)
   (thermal_bridge_angle 0))
  (pad "55" smd roundrect (at 50.7 -1.35) (size 0.6 2.4) (layers "B.Cu") (roundrect_rratio 0.25) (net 45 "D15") (solder_mask_margin 0.1016)
   (thermal_bridge_angle 0))
  (pad "56" smd roundrect (at 51.1 -1.35) (size 0.6 2.4) (layers "F.Cu") (roundrect_rratio 0.25) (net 44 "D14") (solder_mask_margin 0.1016)
   (thermal_bridge_angle 0))
  (pad "56" smd roundrect (at 51.5 -1.35) (size 0.6 2.4) (layers "B.Cu") (roundrect_rratio 0.25) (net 44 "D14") (solder_mask_margin 0.1016)
   (thermal_bridge_angle 0))
  (pad "57" smd roundrect (at 51.9 -1.35) (size 0.6 2.4) (layers "F.Cu") (roundrect_rratio 0.25) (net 13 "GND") (solder_mask_margin 0.1016)
   (thermal_bridge_angle 0))
  (pad "57" smd roundrect (at 52.3 -1.35) (size 0.6 2.4) (layers "B.Cu") (roundrect_rratio 0.25) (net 13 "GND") (solder_mask_margin 0.1016)
   (thermal_bridge_angle 0))
  (pad "58" smd roundrect (at 52.7 -1.35) (size 0.6 2.4) (layers "F.Cu") (roundrect_rratio 0.25) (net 12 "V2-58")
   (solder_mask_margin 0.1016) (thermal_bridge_angle 0))
  (pad "58" smd roundrect (at 53.1 -1.35) (size 0.6 2.4) (layers "B.Cu") (roundrect_rratio 0.25) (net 12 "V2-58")
   (solder_mask_margin 0.1016) (thermal_bridge_angle 0))
  (pad "59" smd roundrect (at 53.5 -1.35) (size 0.6 2.4) (layers "F.Cu") (roundrect_rratio 0.25) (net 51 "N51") (solder_mask_margin 0.1016)
   (thermal_bridge_angle 0))
  (pad "59" smd roundrect (at 53.9 -1.35) (size 0.6 2.4) (layers "B.Cu") (roundrect_rratio 0.25) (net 51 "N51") (solder_mask_margin 0.1016)
   (thermal_bridge_angle 0))
  (pad "60" smd roundrect (at 54.3 -1.35) (size 0.6 2.4) (layers "F.Cu") (roundrect_rratio 0.25) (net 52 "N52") (solder_mask_margin 0.1016)
   (thermal_bridge_angle 0))
  (pad "60" smd roundrect (at 54.7 -1.35) (size 0.6 2.4) (layers "B.Cu") (roundrect_rratio 0.25) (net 52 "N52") (solder_mask_margin 0.1016)
   (thermal_bridge_angle 0))
  (pad "61" smd roundrect (at 55.1 -1.35) (size 0.6 2.4) (layers "F.Cu") (roundrect_rratio 0.25) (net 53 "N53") (solder_mask_margin 0.1016)
   (thermal_bridge_angle 0))
  (pad "61" smd roundrect (at 55.5 -1.35) (size 0.6 2.4) (layers "B.Cu") (roundrect_rratio 0.25) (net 53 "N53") (solder_mask_margin 0.1016)
   (thermal_bridge_angle 0))
  (pad "62" smd roundrect (at 55.9 -1.35) (size 0.6 2.4) (layers "F.Cu") (roundrect_rratio 0.25) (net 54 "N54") (solder_mask_margin 0.1016)
   (thermal_bridge_angle 0))
  (pad "62" smd roundrect (at 56.3 -1.35) (size 0.6 2.4) (layers "B.Cu") (roundrect_rratio 0.25) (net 54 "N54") (solder_mask_margin 0.1016)
   (thermal_bridge_angle 0))
  (pad "EMC-GND1" smd rect (at 1.19 -16.31) (size 1.62 2.62) (layers "F.Cu") (solder_mask_margin 0.1016) (thermal_bridge_angle 0))
  (pad "EMC-GND2" smd rect (at 58.41 -16.31) (size 1.62 2.62) (layers "F.Cu") (solder_mask_margin 0.1016) (thermal_bridge_angle 0))
  (pad "EMC-GND3" smd rect (at 1.19 -10.935) (size 1.62 2.62) (layers "B.Cu") (solder_mask_margin 0.1016) (thermal_bridge_angle 0))
  (pad "EMC-GND4" smd rect (at 58.41 -10.935) (size 1.62 2.62) (layers "B.Cu") (solder_mask_margin 0.1016) (thermal_bridge_angle 0)))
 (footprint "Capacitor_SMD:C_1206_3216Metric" (layer "B.Cu") (at 162.5 92.5)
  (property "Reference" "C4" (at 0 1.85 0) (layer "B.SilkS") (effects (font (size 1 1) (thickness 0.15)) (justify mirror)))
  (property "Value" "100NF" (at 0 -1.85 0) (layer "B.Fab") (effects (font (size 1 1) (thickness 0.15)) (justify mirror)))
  (pad "1" smd roundrect (at -1.475 0) (size 1.15 1.8) (layers "B.Cu" "B.Paste" "B.Mask") (roundrect_rratio 0.217391) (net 35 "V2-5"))
  (pad "2" smd roundrect (at 1.475 0) (size 1.15 1.8) (layers "B.Cu" "B.Paste" "B.Mask") (roundrect_rratio 0.217391) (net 13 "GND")))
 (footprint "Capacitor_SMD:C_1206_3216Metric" (layer "B.Cu") (at 146 132.5 180)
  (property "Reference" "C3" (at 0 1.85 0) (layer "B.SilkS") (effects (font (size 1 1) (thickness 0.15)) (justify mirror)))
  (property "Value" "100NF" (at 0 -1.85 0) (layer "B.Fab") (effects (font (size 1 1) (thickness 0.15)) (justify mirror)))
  (pad "1" smd roundrect (at -1.475 0 180) (size 1.15 1.8) (layers "B.Cu" "B.Paste" "B.Mask") (roundrect_rratio 0.217391) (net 13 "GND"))
  (pad "2" smd roundrect (at 1.475 0 180) (size 1.15 1.8) (layers "B.Cu" "B.Paste" "B.Mask") (roundrect_rratio 0.217391) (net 35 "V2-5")))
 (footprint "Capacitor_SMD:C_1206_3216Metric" (layer "B.Cu") (at 162.5 103)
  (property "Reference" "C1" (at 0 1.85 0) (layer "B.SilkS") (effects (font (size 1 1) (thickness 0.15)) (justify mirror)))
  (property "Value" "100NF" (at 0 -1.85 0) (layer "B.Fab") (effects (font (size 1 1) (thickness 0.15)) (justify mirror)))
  (pad "1" smd roundrect (at -1.475 0) (size 1.15 1.8) (layers "B.Cu" "B.Paste" "B.Mask") (roundrect_rratio 0.217391) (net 12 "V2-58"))
  (pad "2" smd roundrect (at 1.475 0) (size 1.15 1.8) (layers "B.Cu" "B.Paste" "B.Mask") (roundrect_rratio 0.217391) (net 13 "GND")))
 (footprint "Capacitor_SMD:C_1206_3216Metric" (layer "B.Cu") (at 164.5 133)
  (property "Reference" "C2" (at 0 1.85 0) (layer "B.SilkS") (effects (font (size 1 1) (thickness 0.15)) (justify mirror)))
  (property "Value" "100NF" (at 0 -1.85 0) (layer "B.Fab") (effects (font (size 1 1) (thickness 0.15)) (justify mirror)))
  (pad "1" smd roundrect (at -1.475 0) (size 1.15 1.8) (layers "B.Cu" "B.Paste" "B.Mask") (roundrect_rratio 0.217391) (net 13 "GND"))
  (pad "2" smd roundrect (at 1.475 0) (size 1.15 1.8) (layers "B.Cu" "B.Paste" "B.Mask") (roundrect_rratio 0.217391) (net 12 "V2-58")))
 (segment (start 163.975 92.5) (end 163.975 103) (width 0.2) (layer "B.Cu") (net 13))
 (segment (start 166.1 105.125) (end 166.1 105.5) (width 0.2) (layer "B.Cu") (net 13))
 (segment (start 163.975 103) (end 166.1 105.125) (width 0.2) (layer "B.Cu") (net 13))
 (segment (start 162.45 132.425) (end 162.45 104.525) (width 0.2) (layer "B.Cu") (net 13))
 (segment (start 163.025 133) (end 162.45 132.425) (width 0.2) (layer "B.Cu") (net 13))
 (segment (start 162.45 104.525) (end 163.975 103) (width 0.2) (layer "B.Cu") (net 13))
 (segment (start 163.84 110.34) (end 163.84 105.5) (width 0.2) (layer "B.Cu") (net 12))
 (segment (start 165.975 133) (end 165.975 112.475) (width 0.2) (layer "B.Cu") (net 12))
 (segment (start 165.975 112.475) (end 163.84 110.34) (width 0.2) (layer "B.Cu") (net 12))
 (segment (start 149.5 126.5) (end 144.525 131.475) (width 0.2) (layer "B.Cu") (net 35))
 (segment (start 149.5 104.025) (end 149.5 126.5) (width 0.2) (layer "B.Cu") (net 35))
 (segment (start 144.525 131.475) (end 144.525 132.5) (width 0.2) (layer "B.Cu") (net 35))
 (segment (start 161.025 92.5) (end 149.5 104.025) (width 0.2) (layer "B.Cu") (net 35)))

